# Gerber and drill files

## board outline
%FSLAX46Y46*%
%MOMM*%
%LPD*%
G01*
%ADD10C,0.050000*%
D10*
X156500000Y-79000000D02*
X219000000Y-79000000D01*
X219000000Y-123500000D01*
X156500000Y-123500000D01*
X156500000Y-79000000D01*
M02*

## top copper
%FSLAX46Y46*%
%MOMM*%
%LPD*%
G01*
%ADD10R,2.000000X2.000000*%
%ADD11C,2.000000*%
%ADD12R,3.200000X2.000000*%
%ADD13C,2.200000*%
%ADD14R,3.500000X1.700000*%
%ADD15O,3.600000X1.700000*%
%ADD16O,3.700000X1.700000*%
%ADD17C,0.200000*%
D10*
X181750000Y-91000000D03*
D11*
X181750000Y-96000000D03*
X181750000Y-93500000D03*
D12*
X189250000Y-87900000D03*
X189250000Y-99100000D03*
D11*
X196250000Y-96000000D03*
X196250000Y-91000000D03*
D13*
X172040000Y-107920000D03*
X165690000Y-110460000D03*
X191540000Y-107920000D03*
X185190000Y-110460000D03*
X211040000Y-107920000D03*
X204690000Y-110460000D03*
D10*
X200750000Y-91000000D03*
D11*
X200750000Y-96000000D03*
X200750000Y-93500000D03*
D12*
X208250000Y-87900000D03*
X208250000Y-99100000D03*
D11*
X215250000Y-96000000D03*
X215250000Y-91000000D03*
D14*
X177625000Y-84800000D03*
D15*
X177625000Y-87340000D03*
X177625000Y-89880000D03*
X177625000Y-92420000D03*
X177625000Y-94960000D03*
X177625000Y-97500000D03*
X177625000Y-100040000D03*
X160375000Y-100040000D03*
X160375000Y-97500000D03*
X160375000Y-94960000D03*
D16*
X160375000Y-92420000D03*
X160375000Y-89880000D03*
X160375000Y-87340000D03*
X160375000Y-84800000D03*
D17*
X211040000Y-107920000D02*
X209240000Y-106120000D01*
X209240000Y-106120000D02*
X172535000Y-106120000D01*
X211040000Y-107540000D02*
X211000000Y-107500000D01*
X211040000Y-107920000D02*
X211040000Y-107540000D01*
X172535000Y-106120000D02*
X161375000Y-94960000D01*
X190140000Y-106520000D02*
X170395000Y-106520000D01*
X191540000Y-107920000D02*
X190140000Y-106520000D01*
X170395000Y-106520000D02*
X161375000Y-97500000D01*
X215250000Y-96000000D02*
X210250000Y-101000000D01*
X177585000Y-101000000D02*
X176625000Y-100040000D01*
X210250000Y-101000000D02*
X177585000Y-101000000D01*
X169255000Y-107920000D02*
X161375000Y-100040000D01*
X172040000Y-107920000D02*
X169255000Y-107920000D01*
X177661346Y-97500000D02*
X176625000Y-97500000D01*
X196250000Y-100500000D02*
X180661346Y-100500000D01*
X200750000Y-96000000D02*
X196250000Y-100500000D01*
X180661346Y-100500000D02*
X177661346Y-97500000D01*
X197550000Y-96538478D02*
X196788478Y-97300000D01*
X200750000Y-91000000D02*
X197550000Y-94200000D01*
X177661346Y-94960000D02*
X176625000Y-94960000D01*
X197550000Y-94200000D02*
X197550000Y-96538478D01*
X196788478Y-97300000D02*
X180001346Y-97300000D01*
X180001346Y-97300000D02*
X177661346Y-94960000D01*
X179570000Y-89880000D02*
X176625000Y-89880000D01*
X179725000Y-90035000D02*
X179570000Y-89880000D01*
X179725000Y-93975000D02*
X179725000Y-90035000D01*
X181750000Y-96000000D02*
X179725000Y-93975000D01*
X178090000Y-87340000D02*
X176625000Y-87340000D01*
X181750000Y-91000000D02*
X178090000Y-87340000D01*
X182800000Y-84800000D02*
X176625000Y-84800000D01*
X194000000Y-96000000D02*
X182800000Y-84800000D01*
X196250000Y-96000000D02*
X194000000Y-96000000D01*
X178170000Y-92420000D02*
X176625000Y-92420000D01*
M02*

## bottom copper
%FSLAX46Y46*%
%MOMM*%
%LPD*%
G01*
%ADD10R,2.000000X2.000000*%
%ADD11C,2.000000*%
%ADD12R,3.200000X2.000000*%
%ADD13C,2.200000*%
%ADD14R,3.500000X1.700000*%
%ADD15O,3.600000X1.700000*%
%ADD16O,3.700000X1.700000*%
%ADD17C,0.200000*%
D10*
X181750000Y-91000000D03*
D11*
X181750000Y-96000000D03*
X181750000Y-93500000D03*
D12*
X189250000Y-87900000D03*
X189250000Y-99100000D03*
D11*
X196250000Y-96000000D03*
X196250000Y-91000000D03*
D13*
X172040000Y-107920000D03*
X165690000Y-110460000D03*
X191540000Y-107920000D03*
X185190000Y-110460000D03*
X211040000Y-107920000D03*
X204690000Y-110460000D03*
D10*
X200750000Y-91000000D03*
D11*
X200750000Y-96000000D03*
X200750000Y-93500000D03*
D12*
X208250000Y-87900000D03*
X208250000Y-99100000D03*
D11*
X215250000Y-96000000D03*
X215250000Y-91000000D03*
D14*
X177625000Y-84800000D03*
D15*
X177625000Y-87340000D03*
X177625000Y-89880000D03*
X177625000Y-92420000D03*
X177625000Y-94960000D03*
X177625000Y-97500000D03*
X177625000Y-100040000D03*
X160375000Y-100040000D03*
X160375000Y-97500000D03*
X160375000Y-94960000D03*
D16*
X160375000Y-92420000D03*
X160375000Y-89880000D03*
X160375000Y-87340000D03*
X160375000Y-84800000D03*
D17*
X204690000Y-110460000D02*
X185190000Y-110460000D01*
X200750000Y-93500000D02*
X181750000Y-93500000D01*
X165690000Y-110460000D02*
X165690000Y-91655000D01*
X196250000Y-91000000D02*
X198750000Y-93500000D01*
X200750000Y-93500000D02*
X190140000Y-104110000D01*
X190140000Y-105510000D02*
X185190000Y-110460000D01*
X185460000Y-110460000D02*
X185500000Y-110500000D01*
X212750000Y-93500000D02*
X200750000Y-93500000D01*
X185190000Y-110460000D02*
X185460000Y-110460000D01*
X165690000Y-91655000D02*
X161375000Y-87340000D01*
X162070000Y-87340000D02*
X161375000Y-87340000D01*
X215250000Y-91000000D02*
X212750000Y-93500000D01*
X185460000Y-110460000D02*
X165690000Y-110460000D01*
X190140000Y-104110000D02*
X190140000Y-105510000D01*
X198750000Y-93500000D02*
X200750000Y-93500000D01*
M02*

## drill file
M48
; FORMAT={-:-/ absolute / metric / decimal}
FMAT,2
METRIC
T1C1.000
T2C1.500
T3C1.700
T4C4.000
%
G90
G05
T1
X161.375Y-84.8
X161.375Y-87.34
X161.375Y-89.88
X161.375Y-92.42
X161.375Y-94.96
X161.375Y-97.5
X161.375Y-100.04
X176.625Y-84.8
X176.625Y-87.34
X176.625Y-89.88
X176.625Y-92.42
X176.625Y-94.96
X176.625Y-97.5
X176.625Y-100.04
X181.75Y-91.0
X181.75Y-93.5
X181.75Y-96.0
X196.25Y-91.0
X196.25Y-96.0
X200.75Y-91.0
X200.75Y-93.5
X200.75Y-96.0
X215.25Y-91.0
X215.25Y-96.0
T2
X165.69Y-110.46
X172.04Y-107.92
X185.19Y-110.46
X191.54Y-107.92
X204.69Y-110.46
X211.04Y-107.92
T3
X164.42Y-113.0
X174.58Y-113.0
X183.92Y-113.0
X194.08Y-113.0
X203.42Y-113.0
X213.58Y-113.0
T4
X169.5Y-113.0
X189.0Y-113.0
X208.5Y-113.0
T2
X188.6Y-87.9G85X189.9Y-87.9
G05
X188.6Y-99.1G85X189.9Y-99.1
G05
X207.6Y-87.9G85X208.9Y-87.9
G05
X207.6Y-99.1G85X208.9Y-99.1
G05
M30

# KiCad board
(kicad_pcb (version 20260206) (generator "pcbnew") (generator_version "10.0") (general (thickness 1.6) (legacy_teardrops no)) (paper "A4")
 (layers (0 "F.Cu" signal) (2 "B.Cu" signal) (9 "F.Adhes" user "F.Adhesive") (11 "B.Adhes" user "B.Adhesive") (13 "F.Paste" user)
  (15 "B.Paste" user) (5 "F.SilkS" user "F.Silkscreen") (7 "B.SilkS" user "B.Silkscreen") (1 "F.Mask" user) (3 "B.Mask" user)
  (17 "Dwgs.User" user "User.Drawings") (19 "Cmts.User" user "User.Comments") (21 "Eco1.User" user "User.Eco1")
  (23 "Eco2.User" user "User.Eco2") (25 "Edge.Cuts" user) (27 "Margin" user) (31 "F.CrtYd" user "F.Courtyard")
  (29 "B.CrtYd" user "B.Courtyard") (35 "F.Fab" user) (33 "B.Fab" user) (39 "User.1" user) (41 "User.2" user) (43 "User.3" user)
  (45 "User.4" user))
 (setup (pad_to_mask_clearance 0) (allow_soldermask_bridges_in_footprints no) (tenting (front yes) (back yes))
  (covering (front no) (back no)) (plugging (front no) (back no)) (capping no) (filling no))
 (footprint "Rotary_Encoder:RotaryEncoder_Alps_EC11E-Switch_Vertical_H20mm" (layer "F.Cu") (at 181.75 91)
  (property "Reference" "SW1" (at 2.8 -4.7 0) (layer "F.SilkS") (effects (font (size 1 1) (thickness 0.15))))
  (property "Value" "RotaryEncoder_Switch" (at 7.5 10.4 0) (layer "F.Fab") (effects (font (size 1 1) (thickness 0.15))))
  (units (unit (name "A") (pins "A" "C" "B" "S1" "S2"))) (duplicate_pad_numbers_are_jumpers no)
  (pad "A" thru_hole rect (at 0 0) (size 2 2) (drill 1) (layers "*.Cu" "*.Mask") (remove_unused_layers no) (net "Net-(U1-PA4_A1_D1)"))
  (pad "B" thru_hole circle (at 0 5) (size 2 2) (drill 1) (layers "*.Cu" "*.Mask") (remove_unused_layers no) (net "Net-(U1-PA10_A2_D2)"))
  (pad "C" thru_hole circle (at 0 2.5) (size 2 2) (drill 1) (layers "*.Cu" "*.Mask") (remove_unused_layers no) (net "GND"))
  (pad "MP" thru_hole rect (at 7.5 -3.1) (size 3.2 2) (drill oval 2.8 1.5) (layers "*.Cu" "*.Mask") (remove_unused_layers no))
  (pad "MP" thru_hole rect (at 7.5 8.1) (size 3.2 2) (drill oval 2.8 1.5) (layers "*.Cu" "*.Mask") (remove_unused_layers no))
  (pad "S1" thru_hole circle (at 14.5 5) (size 2 2) (drill 1) (layers "*.Cu" "*.Mask") (remove_unused_layers no) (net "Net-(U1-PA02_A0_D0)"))
  (pad "S2" thru_hole circle (at 14.5 0) (size 2 2) (drill 1) (layers "*.Cu" "*.Mask") (remove_unused_layers no) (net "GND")))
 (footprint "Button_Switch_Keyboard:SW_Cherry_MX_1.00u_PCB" (layer "F.Cu") (at 172.04 107.92)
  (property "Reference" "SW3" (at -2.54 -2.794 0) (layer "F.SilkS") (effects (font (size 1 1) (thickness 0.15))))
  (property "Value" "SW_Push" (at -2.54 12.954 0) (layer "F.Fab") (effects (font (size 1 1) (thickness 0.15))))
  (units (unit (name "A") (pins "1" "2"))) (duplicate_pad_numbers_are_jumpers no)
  (pad "" np_thru_hole circle (at -7.62 5.08) (size 1.7 1.7) (drill 1.7) (layers "*.Cu" "*.Mask"))
  (pad "" np_thru_hole circle (at -2.54 5.08) (size 4 4) (drill 4) (layers "*.Cu" "*.Mask"))
  (pad "" np_thru_hole circle (at 2.54 5.08) (size 1.7 1.7) (drill 1.7) (layers "*.Cu" "*.Mask"))
  (pad "1" thru_hole circle (at 0 0) (size 2.2 2.2) (drill 1.5) (layers "*.Cu" "*.Mask") (remove_unused_layers no)
   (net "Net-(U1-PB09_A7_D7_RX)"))
  (pad "2" thru_hole circle (at -6.35 2.54) (size 2.2 2.2) (drill 1.5) (layers "*.Cu" "*.Mask") (remove_unused_layers no) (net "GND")))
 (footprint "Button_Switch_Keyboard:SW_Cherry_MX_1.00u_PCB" (layer "F.Cu") (at 191.54 107.92)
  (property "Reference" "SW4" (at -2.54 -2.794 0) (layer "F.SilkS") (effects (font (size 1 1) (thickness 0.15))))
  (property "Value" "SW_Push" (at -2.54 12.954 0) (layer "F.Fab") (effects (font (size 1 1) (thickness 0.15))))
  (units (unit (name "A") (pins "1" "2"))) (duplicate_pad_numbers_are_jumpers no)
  (pad "" np_thru_hole circle (at -7.62 5.08) (size 1.7 1.7) (drill 1.7) (layers "*.Cu" "*.Mask"))
  (pad "" np_thru_hole circle (at -2.54 5.08) (size 4 4) (drill 4) (layers "*.Cu" "*.Mask"))
  (pad "" np_thru_hole circle (at 2.54 5.08) (size 1.7 1.7) (drill 1.7) (layers "*.Cu" "*.Mask"))
  (pad "1" thru_hole circle (at 0 0) (size 2.2 2.2) (drill 1.5) (layers "*.Cu" "*.Mask") (remove_unused_layers no)
   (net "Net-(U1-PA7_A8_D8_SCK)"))
  (pad "2" thru_hole circle (at -6.35 2.54) (size 2.2 2.2) (drill 1.5) (layers "*.Cu" "*.Mask") (remove_unused_layers no) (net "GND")))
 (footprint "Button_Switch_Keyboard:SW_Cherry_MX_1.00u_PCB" (layer "F.Cu") (at 211.04 107.92)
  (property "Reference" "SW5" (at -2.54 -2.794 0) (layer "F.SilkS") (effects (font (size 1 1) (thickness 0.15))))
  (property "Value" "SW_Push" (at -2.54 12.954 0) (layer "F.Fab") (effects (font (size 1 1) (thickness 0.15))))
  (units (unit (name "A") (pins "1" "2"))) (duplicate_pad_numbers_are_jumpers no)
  (pad "" np_thru_hole circle (at -7.62 5.08) (size 1.7 1.7) (drill 1.7) (layers "*.Cu" "*.Mask"))
  (pad "" np_thru_hole circle (at -2.54 5.08) (size 4 4) (drill 4) (layers "*.Cu" "*.Mask"))
  (pad "" np_thru_hole circle (at 2.54 5.08) (size 1.7 1.7) (drill 1.7) (layers "*.Cu" "*.Mask"))
  (pad "1" thru_hole circle (at 0 0) (size 2.2 2.2) (drill 1.5) (layers "*.Cu" "*.Mask") (remove_unused_layers no)
   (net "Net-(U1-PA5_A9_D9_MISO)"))
  (pad "2" thru_hole circle (at -6.35 2.54) (size 2.2 2.2) (drill 1.5) (layers "*.Cu" "*.Mask") (remove_unused_layers no) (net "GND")))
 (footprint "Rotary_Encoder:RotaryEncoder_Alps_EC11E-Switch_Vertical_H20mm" (layer "F.Cu") (at 200.75 91)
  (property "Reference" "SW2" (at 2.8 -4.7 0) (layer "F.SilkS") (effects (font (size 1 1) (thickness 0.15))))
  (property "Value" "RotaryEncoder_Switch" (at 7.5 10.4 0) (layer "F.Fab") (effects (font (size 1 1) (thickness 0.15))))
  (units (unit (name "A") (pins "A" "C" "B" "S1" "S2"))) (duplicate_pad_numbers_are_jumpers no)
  (pad "A" thru_hole rect (at 0 0) (size 2 2) (drill 1) (layers "*.Cu" "*.Mask") (remove_unused_layers no) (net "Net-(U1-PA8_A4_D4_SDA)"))
  (pad "B" thru_hole circle (at 0 5) (size 2 2) (drill 1) (layers "*.Cu" "*.Mask") (remove_unused_layers no) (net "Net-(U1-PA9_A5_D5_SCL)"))
  (pad "C" thru_hole circle (at 0 2.5) (size 2 2) (drill 1) (layers "*.Cu" "*.Mask") (remove_unused_layers no) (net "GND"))
  (pad "MP" thru_hole rect (at 7.5 -3.1) (size 3.2 2) (drill oval 2.8 1.5) (layers "*.Cu" "*.Mask") (remove_unused_layers no))
  (pad "MP" thru_hole rect (at 7.5 8.1) (size 3.2 2) (drill oval 2.8 1.5) (layers "*.Cu" "*.Mask") (remove_unused_layers no))
  (pad "S1" thru_hole circle (at 14.5 5) (size 2 2) (drill 1) (layers "*.Cu" "*.Mask") (remove_unused_layers no)
   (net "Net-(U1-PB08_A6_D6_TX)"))
  (pad "S2" thru_hole circle (at 14.5 0) (size 2 2) (drill 1) (layers "*.Cu" "*.Mask") (remove_unused_layers no) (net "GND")))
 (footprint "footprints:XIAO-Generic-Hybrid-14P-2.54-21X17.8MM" (layer "B.Cu") (at 169 92.42 180)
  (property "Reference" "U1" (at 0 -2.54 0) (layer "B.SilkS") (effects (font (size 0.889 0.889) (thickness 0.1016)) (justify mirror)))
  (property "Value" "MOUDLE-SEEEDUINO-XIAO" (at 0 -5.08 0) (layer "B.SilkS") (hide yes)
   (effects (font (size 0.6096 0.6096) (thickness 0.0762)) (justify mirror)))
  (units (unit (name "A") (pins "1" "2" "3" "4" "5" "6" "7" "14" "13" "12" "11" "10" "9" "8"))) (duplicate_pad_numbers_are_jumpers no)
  (pad "1" thru_hole rect (at -7.625 7.62 180) (size 3.5 1.7) (drill 1 (offset -1 0)) (layers "*.Cu" "*.Mask") (remove_unused_layers no)
   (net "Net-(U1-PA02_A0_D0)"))
  (pad "2" thru_hole oval (at -7.625 5.08 180) (size 3.6 1.7) (drill 1 (offset -1 0)) (layers "*.Cu" "*.Mask") (remove_unused_layers no)
   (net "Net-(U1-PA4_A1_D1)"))
  (pad "3" thru_hole oval (at -7.625 2.54 180) (size 3.6 1.7) (drill 1 (offset -1 0)) (layers "*.Cu" "*.Mask") (remove_unused_layers no)
   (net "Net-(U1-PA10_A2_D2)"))
  (pad "4" thru_hole oval (at -7.625 0 180) (size 3.6 1.7) (drill 1 (offset -1 0)) (layers "*.Cu" "*.Mask") (remove_unused_layers no)
   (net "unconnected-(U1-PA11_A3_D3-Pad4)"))
  (pad "5" thru_hole oval (at -7.625 -2.54 180) (size 3.6 1.7) (drill 1 (offset -1 0)) (layers "*.Cu" "*.Mask") (remove_unused_layers no)
   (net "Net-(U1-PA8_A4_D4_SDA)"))
  (pad "6" thru_hole oval (at -7.625 -5.08) (size 3.6 1.7) (drill 1 (offset 1 0)) (layers "*.Cu" "*.Mask") (remove_unused_layers no)
   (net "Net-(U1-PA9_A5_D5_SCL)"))
  (pad "7" thru_hole oval (at -7.625 -7.62 180) (size 3.6 1.7) (drill 1 (offset -1 0)) (layers "*.Cu" "*.Mask") (remove_unused_layers no)
   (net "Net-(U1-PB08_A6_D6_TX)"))
  (pad "8" thru_hole oval (at 7.625 -7.62 180) (size 3.6 1.7) (drill 1 (offset 1 0)) (layers "*.Cu" "*.Mask") (remove_unused_layers no)
   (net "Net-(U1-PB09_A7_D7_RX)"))
  (pad "9" thru_hole oval (at 7.625 -5.08 180) (size 3.6 1.7) (drill 1 (offset 1 0)) (layers "*.Cu" "*.Mask") (remove_unused_layers no)
   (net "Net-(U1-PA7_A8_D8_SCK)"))
  (pad "10" thru_hole oval (at 7.625 -2.54 180) (size 3.6 1.7) (drill 1 (offset 1 0)) (layers "*.Cu" "*.Mask") (remove_unused_layers no)
   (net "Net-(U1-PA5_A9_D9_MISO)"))
  (pad "11" thru_hole oval (at 7.625 0 180) (size 3.7 1.7) (drill 1 (offset 1 0)) (layers "*.Cu" "*.Mask") (remove_unused_layers no)
   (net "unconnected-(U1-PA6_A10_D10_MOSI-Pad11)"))
  (pad "12" thru_hole oval (at 7.625 2.54 180) (size 3.7 1.7) (drill 1 (offset 1 0)) (layers "*.Cu" "*.Mask") (remove_unused_layers no)
   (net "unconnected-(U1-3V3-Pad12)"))
  (pad "13" thru_hole oval (at 7.625 5.08 180) (size 3.7 1.7) (drill 1 (offset 1 0)) (layers "*.Cu" "*.Mask") (remove_unused_layers no)
   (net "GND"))
  (pad "14" thru_hole oval (at 7.625 7.62 180) (size 3.7 1.7) (drill 1 (offset 1 0)) (layers "*.Cu" "*.Mask") (remove_unused_layers no)
   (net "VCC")))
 (gr_rect (start 156.5 79) (end 219 123.5) (stroke (width 0.05) (type default)) (fill no) (layer "Edge.Cuts"))
 (segment (start 211.04 107.92) (end 209.24 106.12) (width 0.2) (layer "F.Cu") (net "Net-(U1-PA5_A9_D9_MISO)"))
 (segment (start 209.24 106.12) (end 172.535 106.12) (width 0.2) (layer "F.Cu") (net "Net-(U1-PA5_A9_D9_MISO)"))
 (segment (start 211.04 107.54) (end 211 107.5) (width 0.2) (layer "F.Cu") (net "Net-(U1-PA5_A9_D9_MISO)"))
 (segment (start 211.04 107.92) (end 211.04 107.54) (width 0.2) (layer "F.Cu") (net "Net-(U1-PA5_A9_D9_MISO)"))
 (segment (start 172.535 106.12) (end 161.375 94.96) (width 0.2) (layer "F.Cu") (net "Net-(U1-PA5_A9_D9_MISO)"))
 (segment (start 204.69 110.46) (end 185.19 110.46) (width 0.2) (layer "B.Cu") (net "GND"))
 (segment (start 200.75 93.5) (end 181.75 93.5) (width 0.2) (layer "B.Cu") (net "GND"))
 (segment (start 165.69 110.46) (end 165.69 91.655) (width 0.2) (layer "B.Cu") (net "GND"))
 (segment (start 196.25 91) (end 198.75 93.5) (width 0.2) (layer "B.Cu") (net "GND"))
 (segment (start 200.75 93.5) (end 190.14 104.11) (width 0.2) (layer "B.Cu") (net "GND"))
 (segment (start 190.14 105.51) (end 185.19 110.46) (width 0.2) (layer "B.Cu") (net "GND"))
 (segment (start 185.46 110.46) (end 185.5 110.5) (width 0.2) (layer "B.Cu") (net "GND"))
 (segment (start 212.75 93.5) (end 200.75 93.5) (width 0.2) (layer "B.Cu") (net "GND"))
 (segment (start 185.19 110.46) (end 185.46 110.46) (width 0.2) (layer "B.Cu") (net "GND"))
 (segment (start 165.69 91.655) (end 161.375 87.34) (width 0.2) (layer "B.Cu") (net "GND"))
 (segment (start 162.07 87.34) (end 161.375 87.34) (width 0.2) (layer "B.Cu") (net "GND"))
 (segment (start 215.25 91) (end 212.75 93.5) (width 0.2) (layer "B.Cu") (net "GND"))
 (segment (start 185.46 110.46) (end 165.69 110.46) (width 0.2) (layer "B.Cu") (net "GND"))
 (segment (start 190.14 104.11) (end 190.14 105.51) (width 0.2) (layer "B.Cu") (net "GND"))
 (segment (start 198.75 93.5) (end 200.75 93.5) (width 0.2) (layer "B.Cu") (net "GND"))
 (segment (start 190.14 106.52) (end 170.395 106.52) (width 0.2) (layer "F.Cu") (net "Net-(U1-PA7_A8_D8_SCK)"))
 (segment (start 191.54 107.92) (end 190.14 106.52) (width 0.2) (layer "F.Cu") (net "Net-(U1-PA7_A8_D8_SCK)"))
 (segment (start 170.395 106.52) (end 161.375 97.5) (width 0.2) (layer "F.Cu") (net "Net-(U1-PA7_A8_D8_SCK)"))
 (segment (start 215.25 96) (end 210.25 101) (width 0.2) (layer "F.Cu") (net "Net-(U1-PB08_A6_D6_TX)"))
 (segment (start 177.585 101) (end 176.625 100.04) (width 0.2) (layer "F.Cu") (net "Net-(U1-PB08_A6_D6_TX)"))
 (segment (start 210.25 101) (end 177.585 101) (width 0.2) (layer "F.Cu") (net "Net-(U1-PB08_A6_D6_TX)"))
 (segment (start 169.255 107.92) (end 161.375 100.04) (width 0.2) (layer "F.Cu") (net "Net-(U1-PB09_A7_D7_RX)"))
 (segment (start 172.04 107.92) (end 169.255 107.92) (width 0.2) (layer "F.Cu") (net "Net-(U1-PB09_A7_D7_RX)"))
 (segment (start 177.661346 97.5) (end 176.625 97.5) (width 0.2) (layer "F.Cu") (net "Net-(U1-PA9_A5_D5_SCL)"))
 (segment (start 196.25 100.5) (end 180.661346 100.5) (width 0.2) (layer "F.Cu") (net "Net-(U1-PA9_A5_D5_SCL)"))
 (segment (start 200.75 96) (end 196.25 100.5) (width 0.2) (layer "F.Cu") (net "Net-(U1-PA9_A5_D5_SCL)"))
 (segment (start 180.661346 100.5) (end 177.661346 97.5) (width 0.2) (layer "F.Cu") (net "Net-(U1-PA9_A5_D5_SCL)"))
 (segment (start 197.55 96.538478) (end 196.788478 97.3) (width 0.2) (layer "F.Cu") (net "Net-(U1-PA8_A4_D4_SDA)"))
 (segment (start 200.75 91) (end 197.55 94.2) (width 0.2) (layer "F.Cu") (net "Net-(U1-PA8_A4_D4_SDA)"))
 (segment (start 177.661346 94.96) (end 176.625 94.96) (width 0.2) (layer "F.Cu") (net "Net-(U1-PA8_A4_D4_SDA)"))
 (segment (start 197.55 94.2) (end 197.55 96.538478) (width 0.2) (layer "F.Cu") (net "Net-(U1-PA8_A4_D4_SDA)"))
 (segment (start 196.788478 97.3) (end 180.001346 97.3) (width 0.2) (layer "F.Cu") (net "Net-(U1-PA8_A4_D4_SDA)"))
 (segment (start 180.001346 97.3) (end 177.661346 94.96) (width 0.2) (layer "F.Cu") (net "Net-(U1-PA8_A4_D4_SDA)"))
 (segment (start 179.57 89.88) (end 176.625 89.88) (width 0.2) (layer "F.Cu") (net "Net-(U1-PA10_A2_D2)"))
 (segment (start 179.725 90.035) (end 179.57 89.88) (width 0.2) (layer "F.Cu") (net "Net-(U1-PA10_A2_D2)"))
 (segment (start 179.725 93.975) (end 179.725 90.035) (width 0.2) (layer "F.Cu") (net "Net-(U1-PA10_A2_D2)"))
 (segment (start 181.75 96) (end 179.725 93.975) (width 0.2) (layer "F.Cu") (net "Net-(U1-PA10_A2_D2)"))
 (segment (start 178.09 87.34) (end 176.625 87.34) (width 0.2) (layer "F.Cu") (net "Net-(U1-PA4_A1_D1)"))
 (segment (start 181.75 91) (end 178.09 87.34) (width 0.2) (layer "F.Cu") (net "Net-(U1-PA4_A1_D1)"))
 (segment (start 182.8 84.8) (end 176.625 84.8) (width 0.2) (layer "F.Cu") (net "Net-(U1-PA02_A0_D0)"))
 (segment (start 194 96) (end 182.8 84.8) (width 0.2) (layer "F.Cu") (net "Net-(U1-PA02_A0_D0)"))
 (segment (start 196.25 96) (end 194 96) (width 0.2) (layer "F.Cu") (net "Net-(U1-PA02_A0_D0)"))
 (segment (start 178.17 92.42) (end 176.625 92.42) (width 0.2) (layer "F.Cu") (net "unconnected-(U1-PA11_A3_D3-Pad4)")))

